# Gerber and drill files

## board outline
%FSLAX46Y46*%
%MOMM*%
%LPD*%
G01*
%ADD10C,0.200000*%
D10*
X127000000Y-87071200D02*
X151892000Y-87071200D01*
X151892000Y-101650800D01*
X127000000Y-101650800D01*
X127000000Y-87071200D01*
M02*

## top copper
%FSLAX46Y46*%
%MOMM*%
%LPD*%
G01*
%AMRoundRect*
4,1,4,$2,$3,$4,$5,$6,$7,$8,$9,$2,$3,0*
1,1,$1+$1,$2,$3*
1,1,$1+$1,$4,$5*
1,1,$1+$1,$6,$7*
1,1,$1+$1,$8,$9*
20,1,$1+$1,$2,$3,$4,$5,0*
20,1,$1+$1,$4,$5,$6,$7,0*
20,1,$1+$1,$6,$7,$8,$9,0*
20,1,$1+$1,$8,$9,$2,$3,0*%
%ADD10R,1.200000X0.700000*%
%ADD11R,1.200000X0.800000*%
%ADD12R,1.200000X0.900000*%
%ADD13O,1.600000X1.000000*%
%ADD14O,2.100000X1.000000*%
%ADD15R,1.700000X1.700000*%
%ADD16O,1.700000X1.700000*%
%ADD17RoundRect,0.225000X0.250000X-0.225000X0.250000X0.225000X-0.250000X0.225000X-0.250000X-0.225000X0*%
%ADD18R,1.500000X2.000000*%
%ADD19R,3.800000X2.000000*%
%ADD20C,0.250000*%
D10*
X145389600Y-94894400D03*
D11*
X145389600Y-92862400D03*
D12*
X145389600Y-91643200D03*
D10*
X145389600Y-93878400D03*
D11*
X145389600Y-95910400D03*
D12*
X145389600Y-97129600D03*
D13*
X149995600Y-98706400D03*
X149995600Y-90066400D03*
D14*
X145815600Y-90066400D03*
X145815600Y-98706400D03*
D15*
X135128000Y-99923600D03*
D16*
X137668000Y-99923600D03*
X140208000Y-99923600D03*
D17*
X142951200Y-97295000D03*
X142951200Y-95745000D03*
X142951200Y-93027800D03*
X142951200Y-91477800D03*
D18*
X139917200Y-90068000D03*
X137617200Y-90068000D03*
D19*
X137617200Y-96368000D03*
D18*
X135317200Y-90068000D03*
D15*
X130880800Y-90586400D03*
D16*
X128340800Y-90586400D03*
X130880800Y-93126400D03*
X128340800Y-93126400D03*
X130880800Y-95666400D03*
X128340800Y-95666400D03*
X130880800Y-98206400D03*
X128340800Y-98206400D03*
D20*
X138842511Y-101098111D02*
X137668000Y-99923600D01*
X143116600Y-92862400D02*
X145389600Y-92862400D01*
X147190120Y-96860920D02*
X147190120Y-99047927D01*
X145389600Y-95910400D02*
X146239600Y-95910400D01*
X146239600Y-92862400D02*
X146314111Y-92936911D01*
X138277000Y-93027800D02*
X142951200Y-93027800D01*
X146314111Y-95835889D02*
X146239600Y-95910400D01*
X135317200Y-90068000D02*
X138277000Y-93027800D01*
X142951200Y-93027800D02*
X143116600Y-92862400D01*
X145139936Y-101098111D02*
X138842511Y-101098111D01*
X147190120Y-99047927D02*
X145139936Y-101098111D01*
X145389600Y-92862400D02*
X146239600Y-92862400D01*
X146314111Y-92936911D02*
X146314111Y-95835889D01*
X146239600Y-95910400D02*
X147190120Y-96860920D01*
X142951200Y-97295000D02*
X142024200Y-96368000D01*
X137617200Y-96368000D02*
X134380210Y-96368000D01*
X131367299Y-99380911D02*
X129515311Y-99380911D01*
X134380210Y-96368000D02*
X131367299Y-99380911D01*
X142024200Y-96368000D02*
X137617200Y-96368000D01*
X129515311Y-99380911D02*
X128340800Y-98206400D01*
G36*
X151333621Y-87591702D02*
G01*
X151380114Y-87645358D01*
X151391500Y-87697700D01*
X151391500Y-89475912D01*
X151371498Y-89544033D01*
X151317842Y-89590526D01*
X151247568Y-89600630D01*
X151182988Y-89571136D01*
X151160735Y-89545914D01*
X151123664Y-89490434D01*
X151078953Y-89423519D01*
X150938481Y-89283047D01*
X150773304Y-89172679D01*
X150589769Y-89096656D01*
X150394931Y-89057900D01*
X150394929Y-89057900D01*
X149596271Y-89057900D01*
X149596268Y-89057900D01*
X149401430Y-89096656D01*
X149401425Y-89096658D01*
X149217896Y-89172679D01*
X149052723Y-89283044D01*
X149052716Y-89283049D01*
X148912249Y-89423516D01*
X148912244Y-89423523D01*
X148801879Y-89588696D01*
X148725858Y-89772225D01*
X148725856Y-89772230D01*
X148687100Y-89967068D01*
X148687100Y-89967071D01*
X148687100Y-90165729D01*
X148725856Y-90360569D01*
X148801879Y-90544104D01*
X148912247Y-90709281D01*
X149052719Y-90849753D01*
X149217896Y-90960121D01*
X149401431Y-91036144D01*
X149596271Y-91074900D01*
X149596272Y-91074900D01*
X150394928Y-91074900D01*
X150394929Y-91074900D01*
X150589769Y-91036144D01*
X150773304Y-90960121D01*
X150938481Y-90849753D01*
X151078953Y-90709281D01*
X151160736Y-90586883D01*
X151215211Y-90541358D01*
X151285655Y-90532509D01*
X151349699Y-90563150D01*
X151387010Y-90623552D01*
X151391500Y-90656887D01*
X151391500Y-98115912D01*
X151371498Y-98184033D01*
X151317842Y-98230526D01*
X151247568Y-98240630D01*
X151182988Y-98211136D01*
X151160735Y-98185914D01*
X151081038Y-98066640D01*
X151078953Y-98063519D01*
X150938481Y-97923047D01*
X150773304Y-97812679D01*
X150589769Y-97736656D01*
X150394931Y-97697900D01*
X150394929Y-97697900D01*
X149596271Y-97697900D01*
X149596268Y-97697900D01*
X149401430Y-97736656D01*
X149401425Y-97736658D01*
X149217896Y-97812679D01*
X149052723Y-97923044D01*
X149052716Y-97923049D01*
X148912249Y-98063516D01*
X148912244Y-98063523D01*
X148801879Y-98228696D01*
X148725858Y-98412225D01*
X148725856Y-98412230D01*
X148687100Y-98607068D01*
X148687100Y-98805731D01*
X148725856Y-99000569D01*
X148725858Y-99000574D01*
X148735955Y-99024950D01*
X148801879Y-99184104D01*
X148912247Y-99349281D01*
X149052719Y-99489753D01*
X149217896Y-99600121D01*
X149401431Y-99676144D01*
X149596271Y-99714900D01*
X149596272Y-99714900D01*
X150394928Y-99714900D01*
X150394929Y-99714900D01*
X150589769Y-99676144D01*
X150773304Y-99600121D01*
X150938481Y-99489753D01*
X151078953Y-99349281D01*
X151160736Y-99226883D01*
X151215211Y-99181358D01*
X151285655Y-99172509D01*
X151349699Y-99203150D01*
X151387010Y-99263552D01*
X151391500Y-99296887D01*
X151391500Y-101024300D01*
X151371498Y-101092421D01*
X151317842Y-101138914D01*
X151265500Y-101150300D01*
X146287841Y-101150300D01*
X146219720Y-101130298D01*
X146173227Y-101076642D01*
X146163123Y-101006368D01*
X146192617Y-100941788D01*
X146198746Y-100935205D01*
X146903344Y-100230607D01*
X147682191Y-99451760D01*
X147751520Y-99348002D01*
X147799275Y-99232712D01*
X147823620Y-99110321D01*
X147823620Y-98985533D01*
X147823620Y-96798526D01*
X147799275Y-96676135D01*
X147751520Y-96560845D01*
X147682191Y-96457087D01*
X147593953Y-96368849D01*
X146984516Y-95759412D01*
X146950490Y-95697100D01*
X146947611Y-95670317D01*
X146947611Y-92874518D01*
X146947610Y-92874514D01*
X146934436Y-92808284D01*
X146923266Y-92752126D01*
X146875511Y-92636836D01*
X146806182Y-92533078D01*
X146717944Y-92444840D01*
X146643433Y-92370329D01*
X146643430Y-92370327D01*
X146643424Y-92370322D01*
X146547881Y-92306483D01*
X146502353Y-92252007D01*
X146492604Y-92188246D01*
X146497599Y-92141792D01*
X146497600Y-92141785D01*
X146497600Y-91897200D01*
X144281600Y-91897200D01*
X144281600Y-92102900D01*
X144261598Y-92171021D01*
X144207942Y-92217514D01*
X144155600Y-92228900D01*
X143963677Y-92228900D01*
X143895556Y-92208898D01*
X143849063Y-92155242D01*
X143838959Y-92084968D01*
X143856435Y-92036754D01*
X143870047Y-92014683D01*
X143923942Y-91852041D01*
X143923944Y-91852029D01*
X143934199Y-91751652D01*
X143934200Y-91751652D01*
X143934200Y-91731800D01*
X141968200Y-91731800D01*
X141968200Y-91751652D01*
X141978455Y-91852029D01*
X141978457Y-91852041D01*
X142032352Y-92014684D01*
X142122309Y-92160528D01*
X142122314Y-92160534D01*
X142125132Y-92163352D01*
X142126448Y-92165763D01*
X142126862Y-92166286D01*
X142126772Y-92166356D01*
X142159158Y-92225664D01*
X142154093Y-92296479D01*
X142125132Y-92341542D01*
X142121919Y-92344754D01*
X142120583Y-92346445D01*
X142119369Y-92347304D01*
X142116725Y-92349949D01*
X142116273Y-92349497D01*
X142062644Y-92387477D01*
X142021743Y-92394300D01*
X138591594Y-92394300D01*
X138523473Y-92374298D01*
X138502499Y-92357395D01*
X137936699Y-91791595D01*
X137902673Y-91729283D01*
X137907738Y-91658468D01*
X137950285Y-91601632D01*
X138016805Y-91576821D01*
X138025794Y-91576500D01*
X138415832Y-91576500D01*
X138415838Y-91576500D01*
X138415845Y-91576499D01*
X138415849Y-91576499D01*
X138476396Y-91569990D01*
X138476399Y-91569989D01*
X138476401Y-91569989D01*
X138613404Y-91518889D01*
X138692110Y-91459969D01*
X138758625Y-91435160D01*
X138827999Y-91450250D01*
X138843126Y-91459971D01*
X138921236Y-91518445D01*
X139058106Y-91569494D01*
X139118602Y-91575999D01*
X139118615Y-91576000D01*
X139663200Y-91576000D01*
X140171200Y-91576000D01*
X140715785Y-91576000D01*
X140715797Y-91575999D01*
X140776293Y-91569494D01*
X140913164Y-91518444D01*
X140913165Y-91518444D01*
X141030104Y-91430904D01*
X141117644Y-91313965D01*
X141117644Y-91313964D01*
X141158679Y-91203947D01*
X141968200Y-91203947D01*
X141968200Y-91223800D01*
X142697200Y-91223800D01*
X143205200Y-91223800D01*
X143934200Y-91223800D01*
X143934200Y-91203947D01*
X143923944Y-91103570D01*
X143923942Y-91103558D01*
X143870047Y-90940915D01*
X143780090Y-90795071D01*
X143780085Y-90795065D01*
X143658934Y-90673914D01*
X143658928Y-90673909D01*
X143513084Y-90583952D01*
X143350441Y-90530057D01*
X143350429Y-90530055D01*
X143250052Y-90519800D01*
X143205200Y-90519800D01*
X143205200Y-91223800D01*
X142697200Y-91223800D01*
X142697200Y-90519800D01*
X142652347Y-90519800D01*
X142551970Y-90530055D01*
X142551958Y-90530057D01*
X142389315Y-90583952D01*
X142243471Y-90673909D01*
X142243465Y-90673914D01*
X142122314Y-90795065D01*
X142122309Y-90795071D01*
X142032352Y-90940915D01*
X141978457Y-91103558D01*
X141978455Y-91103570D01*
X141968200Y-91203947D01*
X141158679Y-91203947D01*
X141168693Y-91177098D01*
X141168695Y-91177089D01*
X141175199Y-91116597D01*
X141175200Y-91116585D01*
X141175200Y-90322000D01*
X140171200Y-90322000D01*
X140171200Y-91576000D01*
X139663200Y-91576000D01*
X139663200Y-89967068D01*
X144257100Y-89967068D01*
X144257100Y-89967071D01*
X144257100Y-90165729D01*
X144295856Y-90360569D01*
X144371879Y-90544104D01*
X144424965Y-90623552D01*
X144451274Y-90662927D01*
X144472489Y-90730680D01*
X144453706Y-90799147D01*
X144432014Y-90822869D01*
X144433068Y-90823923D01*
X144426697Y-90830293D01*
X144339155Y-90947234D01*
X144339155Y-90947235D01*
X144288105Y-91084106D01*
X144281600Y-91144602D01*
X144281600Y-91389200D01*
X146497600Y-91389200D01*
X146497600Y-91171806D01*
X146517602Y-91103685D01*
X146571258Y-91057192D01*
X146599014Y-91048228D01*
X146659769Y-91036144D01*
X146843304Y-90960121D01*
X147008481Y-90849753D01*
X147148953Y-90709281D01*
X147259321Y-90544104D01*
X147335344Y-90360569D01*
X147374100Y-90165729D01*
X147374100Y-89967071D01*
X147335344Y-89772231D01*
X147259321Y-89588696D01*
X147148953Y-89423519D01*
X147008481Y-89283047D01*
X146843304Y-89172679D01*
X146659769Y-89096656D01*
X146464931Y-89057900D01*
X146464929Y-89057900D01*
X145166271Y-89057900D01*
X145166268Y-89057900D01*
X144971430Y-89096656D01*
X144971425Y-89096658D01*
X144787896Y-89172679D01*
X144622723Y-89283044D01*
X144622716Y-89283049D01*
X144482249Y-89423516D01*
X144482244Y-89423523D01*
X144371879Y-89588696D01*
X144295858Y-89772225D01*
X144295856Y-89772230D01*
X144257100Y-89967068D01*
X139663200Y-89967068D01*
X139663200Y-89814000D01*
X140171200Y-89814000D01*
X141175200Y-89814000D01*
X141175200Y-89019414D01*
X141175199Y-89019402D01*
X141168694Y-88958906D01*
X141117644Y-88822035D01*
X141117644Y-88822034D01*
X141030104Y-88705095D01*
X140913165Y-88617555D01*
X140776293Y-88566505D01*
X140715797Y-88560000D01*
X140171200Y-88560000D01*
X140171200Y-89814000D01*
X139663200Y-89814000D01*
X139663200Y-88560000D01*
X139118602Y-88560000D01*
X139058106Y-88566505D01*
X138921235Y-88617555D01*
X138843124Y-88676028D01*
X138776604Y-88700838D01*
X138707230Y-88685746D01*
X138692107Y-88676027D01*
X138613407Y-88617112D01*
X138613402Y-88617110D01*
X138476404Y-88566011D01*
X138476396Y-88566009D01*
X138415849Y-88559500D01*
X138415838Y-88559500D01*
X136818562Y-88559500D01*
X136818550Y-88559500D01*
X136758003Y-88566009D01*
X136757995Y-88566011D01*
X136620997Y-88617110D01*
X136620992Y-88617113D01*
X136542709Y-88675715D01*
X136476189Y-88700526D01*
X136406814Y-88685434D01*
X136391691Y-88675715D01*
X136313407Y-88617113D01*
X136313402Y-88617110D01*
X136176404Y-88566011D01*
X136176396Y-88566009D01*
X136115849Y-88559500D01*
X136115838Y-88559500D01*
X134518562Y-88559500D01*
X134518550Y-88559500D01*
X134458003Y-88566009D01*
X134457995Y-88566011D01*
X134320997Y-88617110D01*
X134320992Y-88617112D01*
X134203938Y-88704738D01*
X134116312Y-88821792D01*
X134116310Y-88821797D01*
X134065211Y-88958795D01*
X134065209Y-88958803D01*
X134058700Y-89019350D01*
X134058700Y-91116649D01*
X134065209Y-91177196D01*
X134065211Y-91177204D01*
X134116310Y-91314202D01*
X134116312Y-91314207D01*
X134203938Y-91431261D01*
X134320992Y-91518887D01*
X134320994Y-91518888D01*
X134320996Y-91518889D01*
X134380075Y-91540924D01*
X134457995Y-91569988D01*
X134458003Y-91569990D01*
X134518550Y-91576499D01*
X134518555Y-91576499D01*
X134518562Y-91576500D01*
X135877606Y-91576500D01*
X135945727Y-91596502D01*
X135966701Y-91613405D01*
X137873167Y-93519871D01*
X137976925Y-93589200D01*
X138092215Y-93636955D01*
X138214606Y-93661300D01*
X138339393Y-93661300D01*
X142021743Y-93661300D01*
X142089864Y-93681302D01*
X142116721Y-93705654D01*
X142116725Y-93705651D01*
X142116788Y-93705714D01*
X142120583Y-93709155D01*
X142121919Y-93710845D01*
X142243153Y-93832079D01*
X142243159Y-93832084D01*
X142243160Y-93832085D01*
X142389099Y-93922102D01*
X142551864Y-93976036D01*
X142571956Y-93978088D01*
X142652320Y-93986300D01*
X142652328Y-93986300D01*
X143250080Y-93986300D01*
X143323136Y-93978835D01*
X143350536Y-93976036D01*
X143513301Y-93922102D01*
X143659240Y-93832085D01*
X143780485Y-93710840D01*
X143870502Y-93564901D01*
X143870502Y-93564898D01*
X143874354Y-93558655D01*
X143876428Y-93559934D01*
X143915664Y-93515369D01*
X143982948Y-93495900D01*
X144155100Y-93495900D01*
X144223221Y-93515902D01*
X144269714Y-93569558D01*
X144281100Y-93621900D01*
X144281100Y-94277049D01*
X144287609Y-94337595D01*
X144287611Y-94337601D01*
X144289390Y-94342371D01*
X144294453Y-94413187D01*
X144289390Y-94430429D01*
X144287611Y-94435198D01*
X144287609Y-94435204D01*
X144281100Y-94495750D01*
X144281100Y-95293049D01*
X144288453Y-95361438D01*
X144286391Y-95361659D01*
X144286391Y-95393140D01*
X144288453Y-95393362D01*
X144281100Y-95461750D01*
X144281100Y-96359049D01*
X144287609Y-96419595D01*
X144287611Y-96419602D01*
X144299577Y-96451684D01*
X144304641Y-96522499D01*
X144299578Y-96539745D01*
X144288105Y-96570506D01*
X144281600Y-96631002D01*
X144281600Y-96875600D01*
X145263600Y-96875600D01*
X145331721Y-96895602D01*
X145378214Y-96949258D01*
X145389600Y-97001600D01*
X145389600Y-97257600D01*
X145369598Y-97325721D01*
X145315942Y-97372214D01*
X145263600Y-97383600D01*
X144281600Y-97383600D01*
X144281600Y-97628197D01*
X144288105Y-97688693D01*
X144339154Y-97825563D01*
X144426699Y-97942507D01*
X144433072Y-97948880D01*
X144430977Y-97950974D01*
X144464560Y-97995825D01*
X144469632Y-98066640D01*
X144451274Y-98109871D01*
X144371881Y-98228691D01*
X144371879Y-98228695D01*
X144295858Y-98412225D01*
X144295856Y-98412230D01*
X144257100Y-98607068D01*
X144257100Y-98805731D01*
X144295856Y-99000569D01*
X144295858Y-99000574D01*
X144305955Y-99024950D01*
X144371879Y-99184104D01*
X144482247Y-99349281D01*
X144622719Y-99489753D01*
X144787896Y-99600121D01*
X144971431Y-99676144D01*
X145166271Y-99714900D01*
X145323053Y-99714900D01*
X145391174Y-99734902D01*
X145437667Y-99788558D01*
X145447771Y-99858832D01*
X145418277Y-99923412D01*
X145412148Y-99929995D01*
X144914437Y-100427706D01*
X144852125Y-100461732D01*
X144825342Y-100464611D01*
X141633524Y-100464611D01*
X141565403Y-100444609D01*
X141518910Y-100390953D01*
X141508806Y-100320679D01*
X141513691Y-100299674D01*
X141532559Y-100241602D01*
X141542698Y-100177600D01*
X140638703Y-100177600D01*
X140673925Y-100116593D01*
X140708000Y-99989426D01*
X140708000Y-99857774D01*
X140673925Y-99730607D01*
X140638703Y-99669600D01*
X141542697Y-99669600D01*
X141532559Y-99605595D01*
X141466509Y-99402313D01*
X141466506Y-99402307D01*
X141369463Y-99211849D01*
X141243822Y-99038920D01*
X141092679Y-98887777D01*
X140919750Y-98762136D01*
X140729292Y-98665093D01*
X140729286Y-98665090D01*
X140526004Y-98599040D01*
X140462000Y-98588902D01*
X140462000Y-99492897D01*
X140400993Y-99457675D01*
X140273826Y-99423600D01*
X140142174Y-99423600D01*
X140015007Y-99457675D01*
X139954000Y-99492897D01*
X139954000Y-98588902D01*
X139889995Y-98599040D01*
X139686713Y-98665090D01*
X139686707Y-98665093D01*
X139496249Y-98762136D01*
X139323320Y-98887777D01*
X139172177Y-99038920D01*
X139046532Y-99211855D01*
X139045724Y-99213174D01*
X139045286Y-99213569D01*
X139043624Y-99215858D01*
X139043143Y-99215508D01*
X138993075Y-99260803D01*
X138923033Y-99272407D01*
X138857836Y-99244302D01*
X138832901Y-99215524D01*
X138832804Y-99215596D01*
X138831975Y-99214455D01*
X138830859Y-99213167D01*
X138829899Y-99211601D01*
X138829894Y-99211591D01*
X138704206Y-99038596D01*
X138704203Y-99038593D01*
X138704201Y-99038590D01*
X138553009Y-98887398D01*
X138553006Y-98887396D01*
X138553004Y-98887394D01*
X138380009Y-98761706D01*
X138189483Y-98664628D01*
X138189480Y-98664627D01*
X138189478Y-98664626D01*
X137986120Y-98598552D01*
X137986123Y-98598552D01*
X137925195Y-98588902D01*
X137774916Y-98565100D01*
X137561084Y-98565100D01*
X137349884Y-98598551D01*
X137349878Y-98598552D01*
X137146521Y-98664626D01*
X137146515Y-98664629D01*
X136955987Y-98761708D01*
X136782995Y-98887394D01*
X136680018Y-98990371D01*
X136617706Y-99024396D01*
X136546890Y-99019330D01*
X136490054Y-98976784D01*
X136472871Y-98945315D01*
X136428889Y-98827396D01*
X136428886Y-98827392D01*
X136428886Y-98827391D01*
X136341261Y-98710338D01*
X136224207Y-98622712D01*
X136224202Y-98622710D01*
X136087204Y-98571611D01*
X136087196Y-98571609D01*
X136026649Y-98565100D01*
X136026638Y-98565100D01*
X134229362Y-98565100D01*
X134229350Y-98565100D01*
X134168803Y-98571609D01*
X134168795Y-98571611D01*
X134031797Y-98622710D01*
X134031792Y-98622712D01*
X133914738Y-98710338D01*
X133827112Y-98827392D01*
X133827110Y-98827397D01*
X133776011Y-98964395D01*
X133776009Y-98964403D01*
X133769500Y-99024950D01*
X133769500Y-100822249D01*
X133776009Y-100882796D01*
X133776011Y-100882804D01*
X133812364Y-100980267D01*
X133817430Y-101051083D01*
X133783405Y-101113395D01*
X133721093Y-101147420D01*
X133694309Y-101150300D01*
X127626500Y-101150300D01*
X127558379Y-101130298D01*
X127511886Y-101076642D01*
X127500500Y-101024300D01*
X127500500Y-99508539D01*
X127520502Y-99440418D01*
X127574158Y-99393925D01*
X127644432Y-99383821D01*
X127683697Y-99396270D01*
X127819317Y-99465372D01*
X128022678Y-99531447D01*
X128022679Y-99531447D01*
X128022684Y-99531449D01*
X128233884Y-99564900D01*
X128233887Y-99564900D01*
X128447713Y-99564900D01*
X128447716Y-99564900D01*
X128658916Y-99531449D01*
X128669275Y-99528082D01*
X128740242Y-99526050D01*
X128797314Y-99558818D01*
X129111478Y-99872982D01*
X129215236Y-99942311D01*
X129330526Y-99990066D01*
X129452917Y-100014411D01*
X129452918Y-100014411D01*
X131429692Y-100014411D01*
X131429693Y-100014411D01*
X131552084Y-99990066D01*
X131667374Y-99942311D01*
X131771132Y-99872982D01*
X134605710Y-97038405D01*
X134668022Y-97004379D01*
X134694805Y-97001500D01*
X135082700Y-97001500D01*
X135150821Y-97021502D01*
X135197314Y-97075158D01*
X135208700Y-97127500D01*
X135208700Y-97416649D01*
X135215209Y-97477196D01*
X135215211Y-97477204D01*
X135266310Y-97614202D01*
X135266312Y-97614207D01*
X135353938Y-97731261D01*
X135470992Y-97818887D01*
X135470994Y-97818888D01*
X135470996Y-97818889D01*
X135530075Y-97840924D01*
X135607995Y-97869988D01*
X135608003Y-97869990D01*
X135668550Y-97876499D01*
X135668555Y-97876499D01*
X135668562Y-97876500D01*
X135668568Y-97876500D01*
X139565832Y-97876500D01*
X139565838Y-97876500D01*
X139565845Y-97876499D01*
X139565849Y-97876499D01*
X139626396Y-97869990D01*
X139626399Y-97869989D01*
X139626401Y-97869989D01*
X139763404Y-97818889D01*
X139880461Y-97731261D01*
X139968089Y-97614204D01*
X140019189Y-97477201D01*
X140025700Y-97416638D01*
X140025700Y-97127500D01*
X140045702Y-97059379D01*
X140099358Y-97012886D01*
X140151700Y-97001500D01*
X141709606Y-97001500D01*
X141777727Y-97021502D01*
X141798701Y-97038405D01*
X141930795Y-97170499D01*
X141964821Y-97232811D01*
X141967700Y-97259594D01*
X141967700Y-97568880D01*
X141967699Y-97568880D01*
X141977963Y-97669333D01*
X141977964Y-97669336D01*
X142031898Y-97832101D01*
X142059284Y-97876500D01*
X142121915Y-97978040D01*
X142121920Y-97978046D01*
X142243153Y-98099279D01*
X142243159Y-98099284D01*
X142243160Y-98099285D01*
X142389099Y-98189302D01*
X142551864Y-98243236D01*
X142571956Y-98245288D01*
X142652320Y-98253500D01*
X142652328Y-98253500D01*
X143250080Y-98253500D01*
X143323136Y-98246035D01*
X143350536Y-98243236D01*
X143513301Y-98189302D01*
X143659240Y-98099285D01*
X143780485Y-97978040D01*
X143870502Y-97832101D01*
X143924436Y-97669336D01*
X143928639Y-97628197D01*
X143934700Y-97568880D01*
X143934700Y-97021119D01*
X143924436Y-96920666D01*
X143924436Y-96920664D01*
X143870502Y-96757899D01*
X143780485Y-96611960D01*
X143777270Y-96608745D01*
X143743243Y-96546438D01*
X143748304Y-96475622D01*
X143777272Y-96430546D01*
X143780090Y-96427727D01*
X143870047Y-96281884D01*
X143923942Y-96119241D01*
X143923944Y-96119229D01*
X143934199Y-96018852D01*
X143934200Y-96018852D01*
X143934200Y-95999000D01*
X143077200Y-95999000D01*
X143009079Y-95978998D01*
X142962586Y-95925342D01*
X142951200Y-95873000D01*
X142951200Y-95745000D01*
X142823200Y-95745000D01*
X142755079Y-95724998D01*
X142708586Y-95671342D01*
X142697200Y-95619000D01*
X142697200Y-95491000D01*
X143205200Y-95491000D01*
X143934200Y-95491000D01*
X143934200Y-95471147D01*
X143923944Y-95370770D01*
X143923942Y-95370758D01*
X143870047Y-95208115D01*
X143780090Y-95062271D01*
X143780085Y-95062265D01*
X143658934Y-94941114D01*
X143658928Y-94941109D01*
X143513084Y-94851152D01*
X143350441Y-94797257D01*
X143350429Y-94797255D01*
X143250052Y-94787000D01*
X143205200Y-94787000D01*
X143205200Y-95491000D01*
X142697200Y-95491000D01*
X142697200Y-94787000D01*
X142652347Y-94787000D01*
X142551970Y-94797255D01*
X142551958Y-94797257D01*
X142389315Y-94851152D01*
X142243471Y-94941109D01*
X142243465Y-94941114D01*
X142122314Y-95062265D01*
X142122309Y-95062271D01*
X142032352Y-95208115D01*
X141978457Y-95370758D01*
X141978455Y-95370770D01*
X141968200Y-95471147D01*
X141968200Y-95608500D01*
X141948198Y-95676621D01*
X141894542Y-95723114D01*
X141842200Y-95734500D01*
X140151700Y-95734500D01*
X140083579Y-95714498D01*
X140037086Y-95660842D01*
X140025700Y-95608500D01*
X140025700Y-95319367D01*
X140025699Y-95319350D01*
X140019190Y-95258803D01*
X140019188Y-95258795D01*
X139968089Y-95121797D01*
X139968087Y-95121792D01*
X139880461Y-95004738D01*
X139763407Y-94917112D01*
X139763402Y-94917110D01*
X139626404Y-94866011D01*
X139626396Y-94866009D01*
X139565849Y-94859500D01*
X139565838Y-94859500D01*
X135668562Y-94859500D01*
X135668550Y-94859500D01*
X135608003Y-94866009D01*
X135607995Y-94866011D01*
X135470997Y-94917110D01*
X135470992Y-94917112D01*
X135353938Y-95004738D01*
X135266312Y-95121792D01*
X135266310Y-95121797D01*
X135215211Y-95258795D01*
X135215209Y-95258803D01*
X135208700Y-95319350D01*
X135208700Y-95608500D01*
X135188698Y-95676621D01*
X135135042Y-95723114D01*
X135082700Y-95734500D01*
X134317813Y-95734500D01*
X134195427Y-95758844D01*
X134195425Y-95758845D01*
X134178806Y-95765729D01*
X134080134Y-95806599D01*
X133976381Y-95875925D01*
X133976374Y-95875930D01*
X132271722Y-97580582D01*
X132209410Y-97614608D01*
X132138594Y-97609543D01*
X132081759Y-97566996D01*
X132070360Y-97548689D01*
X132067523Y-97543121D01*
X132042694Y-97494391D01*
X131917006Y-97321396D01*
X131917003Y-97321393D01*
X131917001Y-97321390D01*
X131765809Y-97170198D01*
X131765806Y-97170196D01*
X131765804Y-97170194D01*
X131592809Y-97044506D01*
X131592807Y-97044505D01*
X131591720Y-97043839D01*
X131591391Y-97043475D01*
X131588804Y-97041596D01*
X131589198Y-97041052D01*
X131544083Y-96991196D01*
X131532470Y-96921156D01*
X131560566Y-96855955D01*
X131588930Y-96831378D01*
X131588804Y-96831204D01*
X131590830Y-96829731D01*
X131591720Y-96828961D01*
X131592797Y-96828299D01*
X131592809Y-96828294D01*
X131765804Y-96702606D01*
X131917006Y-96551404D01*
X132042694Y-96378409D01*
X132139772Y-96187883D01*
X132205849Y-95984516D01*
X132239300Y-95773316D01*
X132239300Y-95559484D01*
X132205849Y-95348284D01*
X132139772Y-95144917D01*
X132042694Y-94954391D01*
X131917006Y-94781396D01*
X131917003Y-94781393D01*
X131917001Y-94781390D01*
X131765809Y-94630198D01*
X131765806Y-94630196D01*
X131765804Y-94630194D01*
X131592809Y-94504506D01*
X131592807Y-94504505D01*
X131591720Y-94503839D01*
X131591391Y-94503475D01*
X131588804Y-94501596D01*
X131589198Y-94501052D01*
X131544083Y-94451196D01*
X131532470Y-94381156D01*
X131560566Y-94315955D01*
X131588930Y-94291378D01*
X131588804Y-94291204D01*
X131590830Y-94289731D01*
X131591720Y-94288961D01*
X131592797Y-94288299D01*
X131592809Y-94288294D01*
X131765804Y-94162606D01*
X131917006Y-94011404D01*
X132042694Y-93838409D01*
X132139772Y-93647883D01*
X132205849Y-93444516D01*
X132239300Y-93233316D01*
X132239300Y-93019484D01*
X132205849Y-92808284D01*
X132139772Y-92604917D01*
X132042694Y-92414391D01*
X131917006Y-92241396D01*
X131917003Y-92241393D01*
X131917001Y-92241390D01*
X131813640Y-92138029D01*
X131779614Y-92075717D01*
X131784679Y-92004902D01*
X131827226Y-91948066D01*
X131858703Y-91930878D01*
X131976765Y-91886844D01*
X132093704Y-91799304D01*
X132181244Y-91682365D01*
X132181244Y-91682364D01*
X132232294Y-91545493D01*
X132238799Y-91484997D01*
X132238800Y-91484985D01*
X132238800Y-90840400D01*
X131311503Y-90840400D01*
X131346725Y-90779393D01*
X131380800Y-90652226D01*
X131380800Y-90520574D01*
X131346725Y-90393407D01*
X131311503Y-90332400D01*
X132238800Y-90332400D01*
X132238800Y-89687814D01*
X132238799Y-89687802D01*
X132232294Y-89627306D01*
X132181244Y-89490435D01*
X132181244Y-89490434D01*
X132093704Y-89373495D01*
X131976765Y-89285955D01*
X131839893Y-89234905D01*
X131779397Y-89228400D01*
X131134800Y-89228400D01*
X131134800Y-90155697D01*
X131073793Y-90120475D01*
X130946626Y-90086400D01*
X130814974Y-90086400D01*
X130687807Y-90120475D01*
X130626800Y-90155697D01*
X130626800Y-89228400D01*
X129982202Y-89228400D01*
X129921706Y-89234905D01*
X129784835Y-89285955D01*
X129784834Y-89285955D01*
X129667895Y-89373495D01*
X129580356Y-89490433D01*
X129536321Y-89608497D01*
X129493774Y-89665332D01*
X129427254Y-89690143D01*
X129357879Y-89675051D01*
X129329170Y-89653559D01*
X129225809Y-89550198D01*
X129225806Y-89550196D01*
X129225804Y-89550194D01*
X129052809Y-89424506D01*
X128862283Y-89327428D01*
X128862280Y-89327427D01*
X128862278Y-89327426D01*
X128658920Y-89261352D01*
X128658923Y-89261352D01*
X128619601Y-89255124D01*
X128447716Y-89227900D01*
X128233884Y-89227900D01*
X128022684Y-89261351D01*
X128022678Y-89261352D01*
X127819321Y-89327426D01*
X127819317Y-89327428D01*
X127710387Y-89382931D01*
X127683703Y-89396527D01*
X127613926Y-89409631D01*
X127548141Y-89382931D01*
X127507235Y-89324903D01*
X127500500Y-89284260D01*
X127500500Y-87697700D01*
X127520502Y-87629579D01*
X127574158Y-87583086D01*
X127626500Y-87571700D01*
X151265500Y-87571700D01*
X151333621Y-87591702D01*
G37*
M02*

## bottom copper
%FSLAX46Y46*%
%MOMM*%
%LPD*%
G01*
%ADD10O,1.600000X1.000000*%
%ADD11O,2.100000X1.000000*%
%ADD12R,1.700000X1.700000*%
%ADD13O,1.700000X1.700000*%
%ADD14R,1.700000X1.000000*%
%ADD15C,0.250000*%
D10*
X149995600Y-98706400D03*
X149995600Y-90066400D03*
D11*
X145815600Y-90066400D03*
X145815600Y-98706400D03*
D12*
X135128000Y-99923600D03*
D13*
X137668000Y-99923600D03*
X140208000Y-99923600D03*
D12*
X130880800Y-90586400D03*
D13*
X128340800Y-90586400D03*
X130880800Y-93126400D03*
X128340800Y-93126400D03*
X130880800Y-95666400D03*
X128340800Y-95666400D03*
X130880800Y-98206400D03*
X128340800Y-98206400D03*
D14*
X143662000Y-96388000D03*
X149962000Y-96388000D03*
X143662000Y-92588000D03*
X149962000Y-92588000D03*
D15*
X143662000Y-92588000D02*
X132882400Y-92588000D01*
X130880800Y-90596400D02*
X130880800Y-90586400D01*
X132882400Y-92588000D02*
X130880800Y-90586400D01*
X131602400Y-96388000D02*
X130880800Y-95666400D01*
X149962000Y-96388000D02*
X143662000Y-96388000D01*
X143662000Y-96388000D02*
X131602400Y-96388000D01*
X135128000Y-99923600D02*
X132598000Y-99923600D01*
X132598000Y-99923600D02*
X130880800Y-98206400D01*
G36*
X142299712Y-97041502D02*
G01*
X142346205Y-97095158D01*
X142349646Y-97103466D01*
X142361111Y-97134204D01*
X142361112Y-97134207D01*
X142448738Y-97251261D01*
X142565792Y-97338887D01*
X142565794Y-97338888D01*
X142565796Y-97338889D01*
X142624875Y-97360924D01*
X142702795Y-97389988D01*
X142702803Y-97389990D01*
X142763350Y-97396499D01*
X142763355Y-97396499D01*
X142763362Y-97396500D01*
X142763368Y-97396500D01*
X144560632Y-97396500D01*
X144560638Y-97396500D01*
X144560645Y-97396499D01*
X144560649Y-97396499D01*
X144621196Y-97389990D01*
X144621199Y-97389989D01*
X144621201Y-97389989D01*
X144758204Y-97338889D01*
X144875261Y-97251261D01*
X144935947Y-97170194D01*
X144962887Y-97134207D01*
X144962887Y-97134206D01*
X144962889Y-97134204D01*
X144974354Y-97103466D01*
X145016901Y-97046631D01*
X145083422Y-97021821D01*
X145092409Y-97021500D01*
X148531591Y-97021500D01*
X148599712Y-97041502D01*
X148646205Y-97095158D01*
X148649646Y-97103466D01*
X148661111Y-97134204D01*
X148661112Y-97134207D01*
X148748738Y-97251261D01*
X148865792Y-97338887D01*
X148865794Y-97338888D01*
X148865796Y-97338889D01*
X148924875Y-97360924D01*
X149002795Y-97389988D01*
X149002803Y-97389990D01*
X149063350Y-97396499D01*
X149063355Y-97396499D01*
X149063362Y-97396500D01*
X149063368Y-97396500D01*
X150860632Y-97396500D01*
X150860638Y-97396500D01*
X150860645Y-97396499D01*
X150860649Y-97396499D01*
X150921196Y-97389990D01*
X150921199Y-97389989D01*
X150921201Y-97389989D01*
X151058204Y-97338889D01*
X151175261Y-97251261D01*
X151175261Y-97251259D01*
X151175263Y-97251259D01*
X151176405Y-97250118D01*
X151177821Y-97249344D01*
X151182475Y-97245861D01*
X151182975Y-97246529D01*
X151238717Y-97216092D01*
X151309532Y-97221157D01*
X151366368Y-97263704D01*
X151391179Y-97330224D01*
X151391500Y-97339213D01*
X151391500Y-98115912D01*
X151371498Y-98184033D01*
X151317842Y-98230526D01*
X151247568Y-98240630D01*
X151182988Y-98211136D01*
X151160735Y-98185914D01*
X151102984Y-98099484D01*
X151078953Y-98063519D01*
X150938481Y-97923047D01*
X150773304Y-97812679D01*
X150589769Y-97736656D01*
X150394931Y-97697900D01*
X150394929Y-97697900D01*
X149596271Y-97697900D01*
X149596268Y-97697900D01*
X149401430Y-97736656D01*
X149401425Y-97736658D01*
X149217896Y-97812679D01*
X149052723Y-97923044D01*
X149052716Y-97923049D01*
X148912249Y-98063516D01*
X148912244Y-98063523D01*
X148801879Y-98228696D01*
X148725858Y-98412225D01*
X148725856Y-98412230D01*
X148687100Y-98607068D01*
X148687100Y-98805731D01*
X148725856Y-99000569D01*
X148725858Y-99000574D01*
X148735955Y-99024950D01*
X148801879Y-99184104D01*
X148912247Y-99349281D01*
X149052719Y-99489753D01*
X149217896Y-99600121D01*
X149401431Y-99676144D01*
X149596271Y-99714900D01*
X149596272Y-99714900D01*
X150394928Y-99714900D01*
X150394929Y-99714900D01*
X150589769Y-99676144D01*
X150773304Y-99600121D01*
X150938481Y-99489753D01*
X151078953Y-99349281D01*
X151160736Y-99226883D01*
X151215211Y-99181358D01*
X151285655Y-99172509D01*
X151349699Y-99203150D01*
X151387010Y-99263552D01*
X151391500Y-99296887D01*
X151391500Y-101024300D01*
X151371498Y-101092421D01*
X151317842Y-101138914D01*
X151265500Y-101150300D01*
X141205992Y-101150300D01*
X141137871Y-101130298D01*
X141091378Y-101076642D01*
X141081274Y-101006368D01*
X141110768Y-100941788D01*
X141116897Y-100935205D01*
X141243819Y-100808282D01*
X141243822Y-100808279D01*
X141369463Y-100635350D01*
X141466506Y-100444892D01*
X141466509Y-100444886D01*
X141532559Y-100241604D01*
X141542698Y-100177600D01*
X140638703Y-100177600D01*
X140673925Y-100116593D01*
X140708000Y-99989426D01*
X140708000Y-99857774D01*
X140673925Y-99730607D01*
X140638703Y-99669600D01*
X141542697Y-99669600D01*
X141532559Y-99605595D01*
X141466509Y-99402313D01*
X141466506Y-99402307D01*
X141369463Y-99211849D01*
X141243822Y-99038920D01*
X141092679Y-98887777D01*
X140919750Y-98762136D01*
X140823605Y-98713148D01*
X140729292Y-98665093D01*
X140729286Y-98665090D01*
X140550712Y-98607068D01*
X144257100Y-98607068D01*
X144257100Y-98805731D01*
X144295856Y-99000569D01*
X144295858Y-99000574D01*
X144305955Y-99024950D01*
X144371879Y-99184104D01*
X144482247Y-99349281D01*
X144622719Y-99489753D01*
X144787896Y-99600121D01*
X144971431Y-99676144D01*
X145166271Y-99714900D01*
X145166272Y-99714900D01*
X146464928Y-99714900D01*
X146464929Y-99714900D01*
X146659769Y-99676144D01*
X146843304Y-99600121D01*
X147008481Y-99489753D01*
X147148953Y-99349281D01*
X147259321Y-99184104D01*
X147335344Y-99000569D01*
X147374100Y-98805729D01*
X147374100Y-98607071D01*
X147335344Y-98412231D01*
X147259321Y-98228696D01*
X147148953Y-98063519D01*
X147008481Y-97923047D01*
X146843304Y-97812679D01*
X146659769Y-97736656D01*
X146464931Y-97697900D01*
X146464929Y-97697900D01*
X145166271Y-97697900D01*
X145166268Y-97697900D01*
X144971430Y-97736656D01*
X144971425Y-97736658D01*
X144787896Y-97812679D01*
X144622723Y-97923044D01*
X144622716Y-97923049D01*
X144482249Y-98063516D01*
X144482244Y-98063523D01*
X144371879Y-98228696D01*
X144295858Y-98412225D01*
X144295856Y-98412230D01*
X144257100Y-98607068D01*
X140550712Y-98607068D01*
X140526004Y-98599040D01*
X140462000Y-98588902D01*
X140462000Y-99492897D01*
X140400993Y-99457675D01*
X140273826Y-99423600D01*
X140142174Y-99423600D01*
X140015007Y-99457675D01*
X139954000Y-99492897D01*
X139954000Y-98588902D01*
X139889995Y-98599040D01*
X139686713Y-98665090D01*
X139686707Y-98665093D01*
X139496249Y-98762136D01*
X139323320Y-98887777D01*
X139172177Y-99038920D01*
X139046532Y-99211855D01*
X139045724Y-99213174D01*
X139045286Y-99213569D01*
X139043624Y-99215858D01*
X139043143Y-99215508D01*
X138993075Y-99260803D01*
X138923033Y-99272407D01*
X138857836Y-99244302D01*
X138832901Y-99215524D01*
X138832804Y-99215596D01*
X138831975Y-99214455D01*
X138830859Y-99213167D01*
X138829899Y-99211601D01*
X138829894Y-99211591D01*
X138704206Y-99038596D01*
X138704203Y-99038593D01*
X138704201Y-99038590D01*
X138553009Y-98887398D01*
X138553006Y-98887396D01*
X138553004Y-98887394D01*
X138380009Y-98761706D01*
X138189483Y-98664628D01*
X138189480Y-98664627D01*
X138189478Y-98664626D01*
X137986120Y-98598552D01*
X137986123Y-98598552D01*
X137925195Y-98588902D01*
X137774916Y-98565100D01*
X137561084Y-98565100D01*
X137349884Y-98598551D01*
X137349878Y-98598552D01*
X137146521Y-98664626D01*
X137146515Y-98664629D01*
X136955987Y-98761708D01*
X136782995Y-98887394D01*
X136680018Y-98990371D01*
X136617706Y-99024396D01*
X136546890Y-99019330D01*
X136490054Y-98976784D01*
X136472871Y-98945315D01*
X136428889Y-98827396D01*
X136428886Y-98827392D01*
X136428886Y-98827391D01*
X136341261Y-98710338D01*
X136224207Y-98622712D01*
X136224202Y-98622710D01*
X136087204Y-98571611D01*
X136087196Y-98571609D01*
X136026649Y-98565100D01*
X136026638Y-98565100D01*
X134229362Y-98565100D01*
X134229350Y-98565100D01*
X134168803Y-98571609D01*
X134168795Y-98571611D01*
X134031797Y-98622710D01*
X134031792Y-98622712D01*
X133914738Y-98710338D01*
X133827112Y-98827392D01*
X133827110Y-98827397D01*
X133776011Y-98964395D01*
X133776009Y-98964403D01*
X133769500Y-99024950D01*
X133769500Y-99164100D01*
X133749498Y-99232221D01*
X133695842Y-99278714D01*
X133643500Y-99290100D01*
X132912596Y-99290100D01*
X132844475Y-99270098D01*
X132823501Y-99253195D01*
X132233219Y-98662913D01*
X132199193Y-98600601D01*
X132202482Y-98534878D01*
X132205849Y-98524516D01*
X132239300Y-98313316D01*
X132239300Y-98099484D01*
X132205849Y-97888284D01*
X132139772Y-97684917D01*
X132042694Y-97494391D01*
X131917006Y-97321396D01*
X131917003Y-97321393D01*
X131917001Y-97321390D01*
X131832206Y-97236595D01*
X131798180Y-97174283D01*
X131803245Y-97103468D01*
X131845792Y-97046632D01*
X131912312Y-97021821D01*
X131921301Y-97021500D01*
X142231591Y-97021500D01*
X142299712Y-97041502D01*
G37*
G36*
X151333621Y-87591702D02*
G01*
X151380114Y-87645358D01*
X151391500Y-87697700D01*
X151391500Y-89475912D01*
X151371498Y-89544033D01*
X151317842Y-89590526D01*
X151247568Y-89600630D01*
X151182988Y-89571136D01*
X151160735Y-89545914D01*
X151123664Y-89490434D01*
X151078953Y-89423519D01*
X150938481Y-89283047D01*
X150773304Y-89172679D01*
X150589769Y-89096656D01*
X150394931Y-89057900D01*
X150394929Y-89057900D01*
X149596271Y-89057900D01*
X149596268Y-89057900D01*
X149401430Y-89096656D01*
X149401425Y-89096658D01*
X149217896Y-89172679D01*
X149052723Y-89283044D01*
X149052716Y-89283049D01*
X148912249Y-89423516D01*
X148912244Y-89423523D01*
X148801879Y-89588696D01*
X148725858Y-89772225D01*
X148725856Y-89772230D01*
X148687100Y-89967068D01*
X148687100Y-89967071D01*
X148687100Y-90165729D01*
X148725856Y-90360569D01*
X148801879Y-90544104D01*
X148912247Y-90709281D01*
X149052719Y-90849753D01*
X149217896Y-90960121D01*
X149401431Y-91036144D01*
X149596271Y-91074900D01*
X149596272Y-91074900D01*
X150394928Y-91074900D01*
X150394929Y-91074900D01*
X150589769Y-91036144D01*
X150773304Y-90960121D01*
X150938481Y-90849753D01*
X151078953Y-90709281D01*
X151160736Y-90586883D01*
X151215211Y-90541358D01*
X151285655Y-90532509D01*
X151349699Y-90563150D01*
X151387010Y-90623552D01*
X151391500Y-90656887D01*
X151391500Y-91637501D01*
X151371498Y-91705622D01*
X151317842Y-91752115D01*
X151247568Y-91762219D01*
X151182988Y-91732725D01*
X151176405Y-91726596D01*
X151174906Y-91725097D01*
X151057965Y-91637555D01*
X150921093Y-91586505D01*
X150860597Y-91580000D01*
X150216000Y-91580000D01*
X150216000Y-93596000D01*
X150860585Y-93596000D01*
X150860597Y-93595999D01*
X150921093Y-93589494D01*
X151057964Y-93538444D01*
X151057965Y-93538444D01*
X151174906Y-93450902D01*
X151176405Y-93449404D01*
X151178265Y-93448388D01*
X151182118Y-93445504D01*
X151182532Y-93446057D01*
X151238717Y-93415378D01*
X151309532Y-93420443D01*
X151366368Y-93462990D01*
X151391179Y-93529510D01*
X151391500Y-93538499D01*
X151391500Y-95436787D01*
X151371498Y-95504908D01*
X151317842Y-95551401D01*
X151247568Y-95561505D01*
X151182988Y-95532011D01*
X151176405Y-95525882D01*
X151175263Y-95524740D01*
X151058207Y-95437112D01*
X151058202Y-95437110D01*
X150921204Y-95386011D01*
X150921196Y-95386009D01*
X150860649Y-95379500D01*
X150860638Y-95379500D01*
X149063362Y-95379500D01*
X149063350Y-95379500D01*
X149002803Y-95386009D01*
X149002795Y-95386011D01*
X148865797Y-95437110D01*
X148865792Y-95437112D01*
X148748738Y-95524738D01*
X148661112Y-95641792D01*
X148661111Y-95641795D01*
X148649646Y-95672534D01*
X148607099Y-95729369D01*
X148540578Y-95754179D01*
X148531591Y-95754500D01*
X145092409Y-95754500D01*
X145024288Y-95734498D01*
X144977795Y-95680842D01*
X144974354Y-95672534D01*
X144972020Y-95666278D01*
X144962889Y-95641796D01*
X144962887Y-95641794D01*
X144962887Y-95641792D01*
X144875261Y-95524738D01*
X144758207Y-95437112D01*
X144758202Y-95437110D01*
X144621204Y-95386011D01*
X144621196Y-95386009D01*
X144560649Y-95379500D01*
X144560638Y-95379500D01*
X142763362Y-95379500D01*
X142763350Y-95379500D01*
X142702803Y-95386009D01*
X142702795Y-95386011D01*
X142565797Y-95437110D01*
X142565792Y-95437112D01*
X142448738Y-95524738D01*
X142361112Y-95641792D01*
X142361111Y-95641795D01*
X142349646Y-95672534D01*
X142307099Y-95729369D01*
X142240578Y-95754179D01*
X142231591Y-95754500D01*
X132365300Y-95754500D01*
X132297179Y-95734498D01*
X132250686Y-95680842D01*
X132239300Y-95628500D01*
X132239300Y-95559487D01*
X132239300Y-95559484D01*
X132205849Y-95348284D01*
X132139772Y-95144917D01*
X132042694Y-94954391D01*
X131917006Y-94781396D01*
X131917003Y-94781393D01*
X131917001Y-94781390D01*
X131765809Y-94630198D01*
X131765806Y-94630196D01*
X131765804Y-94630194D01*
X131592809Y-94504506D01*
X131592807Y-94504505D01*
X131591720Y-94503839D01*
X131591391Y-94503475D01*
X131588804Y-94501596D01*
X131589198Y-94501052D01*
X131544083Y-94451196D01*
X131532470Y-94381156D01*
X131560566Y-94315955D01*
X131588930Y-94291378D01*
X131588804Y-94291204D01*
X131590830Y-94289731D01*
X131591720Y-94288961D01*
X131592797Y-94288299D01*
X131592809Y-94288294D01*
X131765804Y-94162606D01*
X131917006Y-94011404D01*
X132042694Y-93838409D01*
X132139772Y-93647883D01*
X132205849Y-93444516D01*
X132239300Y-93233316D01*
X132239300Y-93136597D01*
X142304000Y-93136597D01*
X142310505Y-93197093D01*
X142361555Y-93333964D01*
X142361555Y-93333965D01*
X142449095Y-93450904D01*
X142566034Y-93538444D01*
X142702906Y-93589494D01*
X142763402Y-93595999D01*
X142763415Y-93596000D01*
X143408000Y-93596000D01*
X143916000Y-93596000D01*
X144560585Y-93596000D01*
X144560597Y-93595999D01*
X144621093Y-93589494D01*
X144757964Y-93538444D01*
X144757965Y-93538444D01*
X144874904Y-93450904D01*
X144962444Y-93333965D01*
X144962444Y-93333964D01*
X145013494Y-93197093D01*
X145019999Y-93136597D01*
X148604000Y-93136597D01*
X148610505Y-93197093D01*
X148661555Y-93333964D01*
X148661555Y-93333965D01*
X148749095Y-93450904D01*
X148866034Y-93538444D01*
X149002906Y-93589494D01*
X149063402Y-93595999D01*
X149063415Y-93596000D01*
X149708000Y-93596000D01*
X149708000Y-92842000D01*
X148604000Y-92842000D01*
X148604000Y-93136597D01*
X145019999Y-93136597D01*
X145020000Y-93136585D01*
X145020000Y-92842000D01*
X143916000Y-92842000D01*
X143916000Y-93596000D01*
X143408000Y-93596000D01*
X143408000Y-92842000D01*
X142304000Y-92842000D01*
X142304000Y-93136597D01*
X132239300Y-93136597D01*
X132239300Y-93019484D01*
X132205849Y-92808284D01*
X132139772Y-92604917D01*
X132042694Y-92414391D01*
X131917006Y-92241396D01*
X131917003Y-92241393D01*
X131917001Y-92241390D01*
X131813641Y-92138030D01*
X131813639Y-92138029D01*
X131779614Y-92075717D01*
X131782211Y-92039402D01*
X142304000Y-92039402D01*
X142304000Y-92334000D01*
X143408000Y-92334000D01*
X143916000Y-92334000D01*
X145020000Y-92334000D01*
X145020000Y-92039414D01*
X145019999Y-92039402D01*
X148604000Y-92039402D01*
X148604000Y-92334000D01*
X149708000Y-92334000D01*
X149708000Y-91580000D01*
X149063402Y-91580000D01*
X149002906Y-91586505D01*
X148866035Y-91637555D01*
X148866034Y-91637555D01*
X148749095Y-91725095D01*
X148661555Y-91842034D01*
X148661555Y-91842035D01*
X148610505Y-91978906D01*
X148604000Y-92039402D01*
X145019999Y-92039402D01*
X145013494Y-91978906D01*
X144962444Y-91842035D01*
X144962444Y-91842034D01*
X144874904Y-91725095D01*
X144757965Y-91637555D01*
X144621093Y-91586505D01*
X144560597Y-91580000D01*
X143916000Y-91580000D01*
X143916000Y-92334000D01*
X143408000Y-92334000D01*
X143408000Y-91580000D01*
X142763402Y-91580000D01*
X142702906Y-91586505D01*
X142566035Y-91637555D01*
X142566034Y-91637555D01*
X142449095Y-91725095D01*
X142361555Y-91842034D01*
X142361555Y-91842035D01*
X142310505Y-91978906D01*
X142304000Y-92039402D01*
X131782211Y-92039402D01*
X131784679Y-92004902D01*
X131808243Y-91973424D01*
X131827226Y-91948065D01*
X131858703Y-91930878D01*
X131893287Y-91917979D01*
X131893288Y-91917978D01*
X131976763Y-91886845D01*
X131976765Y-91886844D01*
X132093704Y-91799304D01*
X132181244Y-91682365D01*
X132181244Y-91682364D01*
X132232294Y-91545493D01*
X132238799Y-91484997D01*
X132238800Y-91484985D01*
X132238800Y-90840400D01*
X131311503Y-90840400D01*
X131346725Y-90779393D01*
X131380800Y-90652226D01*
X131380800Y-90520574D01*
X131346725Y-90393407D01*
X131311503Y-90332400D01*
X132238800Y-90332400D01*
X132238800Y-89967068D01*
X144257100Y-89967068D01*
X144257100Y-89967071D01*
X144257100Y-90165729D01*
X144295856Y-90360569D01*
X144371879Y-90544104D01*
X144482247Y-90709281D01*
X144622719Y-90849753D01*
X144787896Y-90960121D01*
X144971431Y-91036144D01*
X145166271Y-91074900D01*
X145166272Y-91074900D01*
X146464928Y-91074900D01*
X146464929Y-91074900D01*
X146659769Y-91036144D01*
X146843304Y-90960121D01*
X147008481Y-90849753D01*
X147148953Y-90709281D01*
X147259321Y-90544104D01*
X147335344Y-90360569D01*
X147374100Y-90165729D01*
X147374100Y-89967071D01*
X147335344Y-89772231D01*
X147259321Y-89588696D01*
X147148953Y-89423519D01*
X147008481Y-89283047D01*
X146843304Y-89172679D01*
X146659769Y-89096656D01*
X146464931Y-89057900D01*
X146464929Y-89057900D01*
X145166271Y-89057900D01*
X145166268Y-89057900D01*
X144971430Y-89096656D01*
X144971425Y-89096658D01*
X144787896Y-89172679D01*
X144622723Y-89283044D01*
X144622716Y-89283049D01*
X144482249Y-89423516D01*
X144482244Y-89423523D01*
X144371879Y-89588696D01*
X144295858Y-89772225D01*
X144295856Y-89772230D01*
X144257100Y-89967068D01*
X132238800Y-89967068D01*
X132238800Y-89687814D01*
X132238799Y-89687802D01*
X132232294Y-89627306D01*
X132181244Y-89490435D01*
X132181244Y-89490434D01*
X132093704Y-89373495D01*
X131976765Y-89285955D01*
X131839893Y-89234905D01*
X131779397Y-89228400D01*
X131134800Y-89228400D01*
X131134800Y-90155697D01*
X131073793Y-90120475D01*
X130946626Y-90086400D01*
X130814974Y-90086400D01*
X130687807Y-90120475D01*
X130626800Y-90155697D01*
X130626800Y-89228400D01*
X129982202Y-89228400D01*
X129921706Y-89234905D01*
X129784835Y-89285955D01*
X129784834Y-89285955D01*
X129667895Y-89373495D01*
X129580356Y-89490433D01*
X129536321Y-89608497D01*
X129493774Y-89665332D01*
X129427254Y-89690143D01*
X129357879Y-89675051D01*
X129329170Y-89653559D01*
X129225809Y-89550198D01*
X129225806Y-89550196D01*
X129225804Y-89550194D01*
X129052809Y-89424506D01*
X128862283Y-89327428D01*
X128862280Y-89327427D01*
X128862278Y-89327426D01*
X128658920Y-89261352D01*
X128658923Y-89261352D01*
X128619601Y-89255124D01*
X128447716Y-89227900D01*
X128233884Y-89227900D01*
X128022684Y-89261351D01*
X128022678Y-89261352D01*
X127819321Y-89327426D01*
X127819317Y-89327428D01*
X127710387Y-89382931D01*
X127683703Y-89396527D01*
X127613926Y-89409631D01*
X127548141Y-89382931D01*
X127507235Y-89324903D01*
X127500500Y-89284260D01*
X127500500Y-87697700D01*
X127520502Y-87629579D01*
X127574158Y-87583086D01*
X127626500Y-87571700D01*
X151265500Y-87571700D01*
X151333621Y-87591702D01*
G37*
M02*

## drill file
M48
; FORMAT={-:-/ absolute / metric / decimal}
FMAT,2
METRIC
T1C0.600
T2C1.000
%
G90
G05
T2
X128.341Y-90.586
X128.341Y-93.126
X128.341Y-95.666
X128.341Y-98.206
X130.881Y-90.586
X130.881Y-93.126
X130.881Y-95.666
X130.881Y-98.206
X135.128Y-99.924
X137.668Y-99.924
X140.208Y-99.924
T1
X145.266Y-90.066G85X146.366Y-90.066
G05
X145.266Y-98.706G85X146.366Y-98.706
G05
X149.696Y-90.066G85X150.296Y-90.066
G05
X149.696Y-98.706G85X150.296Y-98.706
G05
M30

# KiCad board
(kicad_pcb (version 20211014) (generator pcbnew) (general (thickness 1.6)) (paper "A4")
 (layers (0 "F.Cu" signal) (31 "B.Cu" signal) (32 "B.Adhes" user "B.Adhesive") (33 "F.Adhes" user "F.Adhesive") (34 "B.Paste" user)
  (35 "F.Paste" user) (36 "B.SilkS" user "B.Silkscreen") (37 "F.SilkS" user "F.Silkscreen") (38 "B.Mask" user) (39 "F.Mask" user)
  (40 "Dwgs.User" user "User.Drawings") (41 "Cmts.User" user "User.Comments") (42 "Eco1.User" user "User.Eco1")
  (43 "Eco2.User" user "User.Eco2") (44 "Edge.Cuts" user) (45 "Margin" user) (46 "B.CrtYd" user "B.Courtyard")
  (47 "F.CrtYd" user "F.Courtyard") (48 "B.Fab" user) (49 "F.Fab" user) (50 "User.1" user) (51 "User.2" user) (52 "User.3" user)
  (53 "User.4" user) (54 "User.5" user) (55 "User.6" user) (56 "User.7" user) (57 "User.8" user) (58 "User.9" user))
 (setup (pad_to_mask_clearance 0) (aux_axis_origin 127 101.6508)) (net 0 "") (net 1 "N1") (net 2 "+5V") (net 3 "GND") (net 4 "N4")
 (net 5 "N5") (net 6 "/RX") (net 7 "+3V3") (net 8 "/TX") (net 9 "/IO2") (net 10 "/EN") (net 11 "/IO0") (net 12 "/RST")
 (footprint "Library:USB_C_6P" (layer "F.Cu") (at 148.9456 94.3864 90)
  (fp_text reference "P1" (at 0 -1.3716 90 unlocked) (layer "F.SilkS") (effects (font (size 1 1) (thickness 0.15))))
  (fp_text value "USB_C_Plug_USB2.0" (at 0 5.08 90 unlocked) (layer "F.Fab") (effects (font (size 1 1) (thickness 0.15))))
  (pad "A5" smd rect (at -0.508 -3.556 90) (size 0.7 1.2) (layers "F.Cu" "F.Paste" "F.Mask") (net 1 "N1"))
  (pad "A9" smd rect (at 1.524 -3.556 90) (size 0.8 1.2) (layers "F.Cu" "F.Paste" "F.Mask") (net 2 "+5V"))
  (pad "A12" smd rect (at 2.7432 -3.556 90) (size 0.9 1.2) (layers "F.Cu" "F.Paste" "F.Mask") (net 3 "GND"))
  (pad "B5" smd rect (at 0.508 -3.556 90) (size 0.7 1.2) (layers "F.Cu" "F.Paste" "F.Mask") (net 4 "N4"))
  (pad "B9" smd rect (at -1.524 -3.556 90) (size 0.8 1.2) (layers "F.Cu" "F.Paste" "F.Mask") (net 2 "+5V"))
  (pad "B12" smd rect (at -2.7432 -3.556 90) (size 0.9 1.2) (layers "F.Cu" "F.Paste" "F.Mask") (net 3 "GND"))
  (pad "S1" thru_hole oval (at -4.32 1.05 90) (size 1 1.6) (drill oval 0.6 1.2) (layers *.Cu *.Mask) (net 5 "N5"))
  (pad "S1" thru_hole oval (at 4.32 1.05 90) (size 1 1.6) (drill oval 0.6 1.2) (layers *.Cu *.Mask) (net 5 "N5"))
  (pad "S1" thru_hole oval (at 4.32 -3.13 90) (size 1 2.1) (drill oval 0.6 1.7) (layers *.Cu *.Mask) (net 5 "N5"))
  (pad "S1" thru_hole oval (at -4.32 -3.13 90) (size 1 2.1) (drill oval 0.6 1.7) (layers *.Cu *.Mask) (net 5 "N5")))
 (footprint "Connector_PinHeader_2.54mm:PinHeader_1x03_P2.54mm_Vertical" (layer "F.Cu") (at 135.128 99.9236 90)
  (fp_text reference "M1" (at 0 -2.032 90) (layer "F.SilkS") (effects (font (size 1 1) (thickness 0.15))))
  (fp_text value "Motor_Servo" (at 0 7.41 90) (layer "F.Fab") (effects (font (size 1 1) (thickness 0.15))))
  (pad "1" thru_hole rect (at 0 0 90) (size 1.7 1.7) (drill 1) (layers *.Cu *.Mask) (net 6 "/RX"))
  (pad "2" thru_hole oval (at 0 2.54 90) (size 1.7 1.7) (drill 1) (layers *.Cu *.Mask) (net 2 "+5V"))
  (pad "3" thru_hole oval (at 0 5.08 90) (size 1.7 1.7) (drill 1) (layers *.Cu *.Mask) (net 3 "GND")))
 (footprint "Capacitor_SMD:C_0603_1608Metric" (layer "F.Cu") (at 142.9512 96.52 90)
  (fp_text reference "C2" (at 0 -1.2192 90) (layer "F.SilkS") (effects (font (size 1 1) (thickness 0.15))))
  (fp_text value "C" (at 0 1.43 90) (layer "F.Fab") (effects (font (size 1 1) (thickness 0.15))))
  (pad "1" smd roundrect (at -0.775 0 90) (size 0.9 0.95) (layers "F.Cu" "F.Paste" "F.Mask") (roundrect_rratio 0.25) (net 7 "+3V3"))
  (pad "2" smd roundrect (at 0.775 0 90) (size 0.9 0.95) (layers "F.Cu" "F.Paste" "F.Mask") (roundrect_rratio 0.25) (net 3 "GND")))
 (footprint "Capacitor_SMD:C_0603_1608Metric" (layer "F.Cu") (at 142.9512 92.2528 90)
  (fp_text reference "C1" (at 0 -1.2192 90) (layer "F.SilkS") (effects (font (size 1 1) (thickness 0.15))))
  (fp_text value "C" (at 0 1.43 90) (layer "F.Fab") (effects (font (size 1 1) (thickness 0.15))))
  (pad "1" smd roundrect (at -0.775 0 90) (size 0.9 0.95) (layers "F.Cu" "F.Paste" "F.Mask") (roundrect_rratio 0.25) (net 2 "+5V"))
  (pad "2" smd roundrect (at 0.775 0 90) (size 0.9 0.95) (layers "F.Cu" "F.Paste" "F.Mask") (roundrect_rratio 0.25) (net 3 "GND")))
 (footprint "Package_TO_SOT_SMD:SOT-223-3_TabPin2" (layer "F.Cu") (at 137.6172 93.218 -90)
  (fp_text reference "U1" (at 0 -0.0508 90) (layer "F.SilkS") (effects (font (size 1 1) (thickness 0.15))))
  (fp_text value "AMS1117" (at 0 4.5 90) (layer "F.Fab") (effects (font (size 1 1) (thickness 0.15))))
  (pad "1" smd rect (at -3.15 -2.3 270) (size 2 1.5) (layers "F.Cu" "F.Paste" "F.Mask") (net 3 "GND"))
  (pad "2" smd rect (at -3.15 0 270) (size 2 1.5) (layers "F.Cu" "F.Paste" "F.Mask") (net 7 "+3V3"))
  (pad "2" smd rect (at 3.15 0 270) (size 2 3.8) (layers "F.Cu" "F.Paste" "F.Mask") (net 7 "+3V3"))
  (pad "3" smd rect (at -3.15 2.3 270) (size 2 1.5) (layers "F.Cu" "F.Paste" "F.Mask") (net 2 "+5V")))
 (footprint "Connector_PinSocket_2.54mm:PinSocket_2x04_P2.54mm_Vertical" (layer "F.Cu") (at 130.8808 90.5864)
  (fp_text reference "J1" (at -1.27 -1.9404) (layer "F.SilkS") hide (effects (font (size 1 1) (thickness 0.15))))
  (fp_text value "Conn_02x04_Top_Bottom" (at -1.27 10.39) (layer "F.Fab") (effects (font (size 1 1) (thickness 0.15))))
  (pad "1" thru_hole rect (at 0 0) (size 1.7 1.7) (drill 1) (layers *.Cu *.Mask) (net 3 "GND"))
  (pad "2" thru_hole oval (at -2.54 0) (size 1.7 1.7) (drill 1) (layers *.Cu *.Mask) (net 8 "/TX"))
  (pad "3" thru_hole oval (at 0 2.54) (size 1.7 1.7) (drill 1) (layers *.Cu *.Mask) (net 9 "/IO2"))
  (pad "4" thru_hole oval (at -2.54 2.54) (size 1.7 1.7) (drill 1) (layers *.Cu *.Mask) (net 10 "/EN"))
  (pad "5" thru_hole oval (at 0 5.08) (size 1.7 1.7) (drill 1) (layers *.Cu *.Mask) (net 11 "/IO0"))
  (pad "6" thru_hole oval (at -2.54 5.08) (size 1.7 1.7) (drill 1) (layers *.Cu *.Mask) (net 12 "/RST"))
  (pad "7" thru_hole oval (at 0 7.62) (size 1.7 1.7) (drill 1) (layers *.Cu *.Mask) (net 6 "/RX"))
  (pad "8" thru_hole oval (at -2.54 7.62) (size 1.7 1.7) (drill 1) (layers *.Cu *.Mask) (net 7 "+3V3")))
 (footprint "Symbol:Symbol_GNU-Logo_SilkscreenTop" (layer "B.Cu") (at 137.922 91.948 180)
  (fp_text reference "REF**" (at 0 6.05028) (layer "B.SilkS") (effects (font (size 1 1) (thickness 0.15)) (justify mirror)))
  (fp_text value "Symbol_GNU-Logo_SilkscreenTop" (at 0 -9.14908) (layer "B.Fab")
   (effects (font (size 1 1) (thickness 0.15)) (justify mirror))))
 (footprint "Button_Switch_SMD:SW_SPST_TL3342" (layer "B.Cu") (at 146.812 94.488)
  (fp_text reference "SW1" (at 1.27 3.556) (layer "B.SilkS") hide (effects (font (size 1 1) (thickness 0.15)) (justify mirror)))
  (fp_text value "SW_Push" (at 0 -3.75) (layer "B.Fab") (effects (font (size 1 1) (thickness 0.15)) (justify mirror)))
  (pad "1" smd rect (at -3.15 1.9) (size 1.7 1) (layers "B.Cu" "B.Paste" "B.Mask") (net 11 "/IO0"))
  (pad "1" smd rect (at 3.15 1.9) (size 1.7 1) (layers "B.Cu" "B.Paste" "B.Mask") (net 11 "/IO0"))
  (pad "2" smd rect (at -3.15 -1.9) (size 1.7 1) (layers "B.Cu" "B.Paste" "B.Mask") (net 3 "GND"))
  (pad "2" smd rect (at 3.15 -1.9) (size 1.7 1) (layers "B.Cu" "B.Paste" "B.Mask") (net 3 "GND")))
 (gr_rect (start 127 101.6508) (end 151.892 87.0712) (layer "Edge.Cuts") (width 0.2) (fill none))
 (segment (start 138.842511 101.098111) (end 137.668 99.9236) (width 0.25) (layer "F.Cu") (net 2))
 (segment (start 143.1166 92.8624) (end 145.3896 92.8624) (width 0.25) (layer "F.Cu") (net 2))
 (segment (start 147.19012 96.86092) (end 147.19012 99.047927) (width 0.25) (layer "F.Cu") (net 2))
 (segment (start 145.3896 95.9104) (end 146.2396 95.9104) (width 0.25) (layer "F.Cu") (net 2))
 (segment (start 146.2396 92.8624) (end 146.314111 92.936911) (width 0.25) (layer "F.Cu") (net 2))
 (segment (start 138.277 93.0278) (end 142.9512 93.0278) (width 0.25) (layer "F.Cu") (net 2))
 (segment (start 146.314111 95.835889) (end 146.2396 95.9104) (width 0.25) (layer "F.Cu") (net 2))
 (segment (start 135.3172 90.068) (end 138.277 93.0278) (width 0.25) (layer "F.Cu") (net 2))
 (segment (start 142.9512 93.0278) (end 143.1166 92.8624) (width 0.25) (layer "F.Cu") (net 2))
 (segment (start 145.139936 101.098111) (end 138.842511 101.098111) (width 0.25) (layer "F.Cu") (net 2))
 (segment (start 147.19012 99.047927) (end 145.139936 101.098111) (width 0.25) (layer "F.Cu") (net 2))
 (segment (start 145.3896 92.8624) (end 146.2396 92.8624) (width 0.25) (layer "F.Cu") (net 2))
 (segment (start 146.314111 92.936911) (end 146.314111 95.835889) (width 0.25) (layer "F.Cu") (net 2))
 (segment (start 146.2396 95.9104) (end 147.19012 96.86092) (width 0.25) (layer "F.Cu") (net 2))
 (segment (start 143.662 92.588) (end 132.8824 92.588) (width 0.25) (layer "B.Cu") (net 3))
 (segment (start 130.8808 90.5964) (end 130.8808 90.5864) (width 0.25) (layer "B.Cu") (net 3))
 (segment (start 132.8824 92.588) (end 130.8808 90.5864) (width 0.25) (layer "B.Cu") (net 3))
 (segment (start 142.9512 97.295) (end 142.0242 96.368) (width 0.25) (layer "F.Cu") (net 7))
 (segment (start 137.6172 96.368) (end 134.38021 96.368) (width 0.25) (layer "F.Cu") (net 7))
 (segment (start 131.367299 99.380911) (end 129.515311 99.380911) (width 0.25) (layer "F.Cu") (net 7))
 (segment (start 134.38021 96.368) (end 131.367299 99.380911) (width 0.25) (layer "F.Cu") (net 7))
 (segment (start 142.0242 96.368) (end 137.6172 96.368) (width 0.25) (layer "F.Cu") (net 7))
 (segment (start 129.515311 99.380911) (end 128.3408 98.2064) (width 0.25) (layer "F.Cu") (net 7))
 (segment (start 131.6024 96.388) (end 130.8808 95.6664) (width 0.25) (layer "B.Cu") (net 11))
 (segment (start 149.962 96.388) (end 143.662 96.388) (width 0.25) (layer "B.Cu") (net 11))
 (segment (start 143.662 96.388) (end 131.6024 96.388) (width 0.25) (layer "B.Cu") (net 11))
 (segment (start 135.128 99.9236) (end 132.598 99.9236) (width 0.25) (layer "B.Cu") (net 6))
 (segment (start 132.598 99.9236) (end 130.8808 98.2064) (width 0.25) (layer "B.Cu") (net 6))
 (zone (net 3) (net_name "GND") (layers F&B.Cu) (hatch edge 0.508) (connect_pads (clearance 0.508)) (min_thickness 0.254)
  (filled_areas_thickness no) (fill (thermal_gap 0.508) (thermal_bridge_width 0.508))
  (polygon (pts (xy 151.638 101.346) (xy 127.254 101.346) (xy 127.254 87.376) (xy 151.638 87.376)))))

